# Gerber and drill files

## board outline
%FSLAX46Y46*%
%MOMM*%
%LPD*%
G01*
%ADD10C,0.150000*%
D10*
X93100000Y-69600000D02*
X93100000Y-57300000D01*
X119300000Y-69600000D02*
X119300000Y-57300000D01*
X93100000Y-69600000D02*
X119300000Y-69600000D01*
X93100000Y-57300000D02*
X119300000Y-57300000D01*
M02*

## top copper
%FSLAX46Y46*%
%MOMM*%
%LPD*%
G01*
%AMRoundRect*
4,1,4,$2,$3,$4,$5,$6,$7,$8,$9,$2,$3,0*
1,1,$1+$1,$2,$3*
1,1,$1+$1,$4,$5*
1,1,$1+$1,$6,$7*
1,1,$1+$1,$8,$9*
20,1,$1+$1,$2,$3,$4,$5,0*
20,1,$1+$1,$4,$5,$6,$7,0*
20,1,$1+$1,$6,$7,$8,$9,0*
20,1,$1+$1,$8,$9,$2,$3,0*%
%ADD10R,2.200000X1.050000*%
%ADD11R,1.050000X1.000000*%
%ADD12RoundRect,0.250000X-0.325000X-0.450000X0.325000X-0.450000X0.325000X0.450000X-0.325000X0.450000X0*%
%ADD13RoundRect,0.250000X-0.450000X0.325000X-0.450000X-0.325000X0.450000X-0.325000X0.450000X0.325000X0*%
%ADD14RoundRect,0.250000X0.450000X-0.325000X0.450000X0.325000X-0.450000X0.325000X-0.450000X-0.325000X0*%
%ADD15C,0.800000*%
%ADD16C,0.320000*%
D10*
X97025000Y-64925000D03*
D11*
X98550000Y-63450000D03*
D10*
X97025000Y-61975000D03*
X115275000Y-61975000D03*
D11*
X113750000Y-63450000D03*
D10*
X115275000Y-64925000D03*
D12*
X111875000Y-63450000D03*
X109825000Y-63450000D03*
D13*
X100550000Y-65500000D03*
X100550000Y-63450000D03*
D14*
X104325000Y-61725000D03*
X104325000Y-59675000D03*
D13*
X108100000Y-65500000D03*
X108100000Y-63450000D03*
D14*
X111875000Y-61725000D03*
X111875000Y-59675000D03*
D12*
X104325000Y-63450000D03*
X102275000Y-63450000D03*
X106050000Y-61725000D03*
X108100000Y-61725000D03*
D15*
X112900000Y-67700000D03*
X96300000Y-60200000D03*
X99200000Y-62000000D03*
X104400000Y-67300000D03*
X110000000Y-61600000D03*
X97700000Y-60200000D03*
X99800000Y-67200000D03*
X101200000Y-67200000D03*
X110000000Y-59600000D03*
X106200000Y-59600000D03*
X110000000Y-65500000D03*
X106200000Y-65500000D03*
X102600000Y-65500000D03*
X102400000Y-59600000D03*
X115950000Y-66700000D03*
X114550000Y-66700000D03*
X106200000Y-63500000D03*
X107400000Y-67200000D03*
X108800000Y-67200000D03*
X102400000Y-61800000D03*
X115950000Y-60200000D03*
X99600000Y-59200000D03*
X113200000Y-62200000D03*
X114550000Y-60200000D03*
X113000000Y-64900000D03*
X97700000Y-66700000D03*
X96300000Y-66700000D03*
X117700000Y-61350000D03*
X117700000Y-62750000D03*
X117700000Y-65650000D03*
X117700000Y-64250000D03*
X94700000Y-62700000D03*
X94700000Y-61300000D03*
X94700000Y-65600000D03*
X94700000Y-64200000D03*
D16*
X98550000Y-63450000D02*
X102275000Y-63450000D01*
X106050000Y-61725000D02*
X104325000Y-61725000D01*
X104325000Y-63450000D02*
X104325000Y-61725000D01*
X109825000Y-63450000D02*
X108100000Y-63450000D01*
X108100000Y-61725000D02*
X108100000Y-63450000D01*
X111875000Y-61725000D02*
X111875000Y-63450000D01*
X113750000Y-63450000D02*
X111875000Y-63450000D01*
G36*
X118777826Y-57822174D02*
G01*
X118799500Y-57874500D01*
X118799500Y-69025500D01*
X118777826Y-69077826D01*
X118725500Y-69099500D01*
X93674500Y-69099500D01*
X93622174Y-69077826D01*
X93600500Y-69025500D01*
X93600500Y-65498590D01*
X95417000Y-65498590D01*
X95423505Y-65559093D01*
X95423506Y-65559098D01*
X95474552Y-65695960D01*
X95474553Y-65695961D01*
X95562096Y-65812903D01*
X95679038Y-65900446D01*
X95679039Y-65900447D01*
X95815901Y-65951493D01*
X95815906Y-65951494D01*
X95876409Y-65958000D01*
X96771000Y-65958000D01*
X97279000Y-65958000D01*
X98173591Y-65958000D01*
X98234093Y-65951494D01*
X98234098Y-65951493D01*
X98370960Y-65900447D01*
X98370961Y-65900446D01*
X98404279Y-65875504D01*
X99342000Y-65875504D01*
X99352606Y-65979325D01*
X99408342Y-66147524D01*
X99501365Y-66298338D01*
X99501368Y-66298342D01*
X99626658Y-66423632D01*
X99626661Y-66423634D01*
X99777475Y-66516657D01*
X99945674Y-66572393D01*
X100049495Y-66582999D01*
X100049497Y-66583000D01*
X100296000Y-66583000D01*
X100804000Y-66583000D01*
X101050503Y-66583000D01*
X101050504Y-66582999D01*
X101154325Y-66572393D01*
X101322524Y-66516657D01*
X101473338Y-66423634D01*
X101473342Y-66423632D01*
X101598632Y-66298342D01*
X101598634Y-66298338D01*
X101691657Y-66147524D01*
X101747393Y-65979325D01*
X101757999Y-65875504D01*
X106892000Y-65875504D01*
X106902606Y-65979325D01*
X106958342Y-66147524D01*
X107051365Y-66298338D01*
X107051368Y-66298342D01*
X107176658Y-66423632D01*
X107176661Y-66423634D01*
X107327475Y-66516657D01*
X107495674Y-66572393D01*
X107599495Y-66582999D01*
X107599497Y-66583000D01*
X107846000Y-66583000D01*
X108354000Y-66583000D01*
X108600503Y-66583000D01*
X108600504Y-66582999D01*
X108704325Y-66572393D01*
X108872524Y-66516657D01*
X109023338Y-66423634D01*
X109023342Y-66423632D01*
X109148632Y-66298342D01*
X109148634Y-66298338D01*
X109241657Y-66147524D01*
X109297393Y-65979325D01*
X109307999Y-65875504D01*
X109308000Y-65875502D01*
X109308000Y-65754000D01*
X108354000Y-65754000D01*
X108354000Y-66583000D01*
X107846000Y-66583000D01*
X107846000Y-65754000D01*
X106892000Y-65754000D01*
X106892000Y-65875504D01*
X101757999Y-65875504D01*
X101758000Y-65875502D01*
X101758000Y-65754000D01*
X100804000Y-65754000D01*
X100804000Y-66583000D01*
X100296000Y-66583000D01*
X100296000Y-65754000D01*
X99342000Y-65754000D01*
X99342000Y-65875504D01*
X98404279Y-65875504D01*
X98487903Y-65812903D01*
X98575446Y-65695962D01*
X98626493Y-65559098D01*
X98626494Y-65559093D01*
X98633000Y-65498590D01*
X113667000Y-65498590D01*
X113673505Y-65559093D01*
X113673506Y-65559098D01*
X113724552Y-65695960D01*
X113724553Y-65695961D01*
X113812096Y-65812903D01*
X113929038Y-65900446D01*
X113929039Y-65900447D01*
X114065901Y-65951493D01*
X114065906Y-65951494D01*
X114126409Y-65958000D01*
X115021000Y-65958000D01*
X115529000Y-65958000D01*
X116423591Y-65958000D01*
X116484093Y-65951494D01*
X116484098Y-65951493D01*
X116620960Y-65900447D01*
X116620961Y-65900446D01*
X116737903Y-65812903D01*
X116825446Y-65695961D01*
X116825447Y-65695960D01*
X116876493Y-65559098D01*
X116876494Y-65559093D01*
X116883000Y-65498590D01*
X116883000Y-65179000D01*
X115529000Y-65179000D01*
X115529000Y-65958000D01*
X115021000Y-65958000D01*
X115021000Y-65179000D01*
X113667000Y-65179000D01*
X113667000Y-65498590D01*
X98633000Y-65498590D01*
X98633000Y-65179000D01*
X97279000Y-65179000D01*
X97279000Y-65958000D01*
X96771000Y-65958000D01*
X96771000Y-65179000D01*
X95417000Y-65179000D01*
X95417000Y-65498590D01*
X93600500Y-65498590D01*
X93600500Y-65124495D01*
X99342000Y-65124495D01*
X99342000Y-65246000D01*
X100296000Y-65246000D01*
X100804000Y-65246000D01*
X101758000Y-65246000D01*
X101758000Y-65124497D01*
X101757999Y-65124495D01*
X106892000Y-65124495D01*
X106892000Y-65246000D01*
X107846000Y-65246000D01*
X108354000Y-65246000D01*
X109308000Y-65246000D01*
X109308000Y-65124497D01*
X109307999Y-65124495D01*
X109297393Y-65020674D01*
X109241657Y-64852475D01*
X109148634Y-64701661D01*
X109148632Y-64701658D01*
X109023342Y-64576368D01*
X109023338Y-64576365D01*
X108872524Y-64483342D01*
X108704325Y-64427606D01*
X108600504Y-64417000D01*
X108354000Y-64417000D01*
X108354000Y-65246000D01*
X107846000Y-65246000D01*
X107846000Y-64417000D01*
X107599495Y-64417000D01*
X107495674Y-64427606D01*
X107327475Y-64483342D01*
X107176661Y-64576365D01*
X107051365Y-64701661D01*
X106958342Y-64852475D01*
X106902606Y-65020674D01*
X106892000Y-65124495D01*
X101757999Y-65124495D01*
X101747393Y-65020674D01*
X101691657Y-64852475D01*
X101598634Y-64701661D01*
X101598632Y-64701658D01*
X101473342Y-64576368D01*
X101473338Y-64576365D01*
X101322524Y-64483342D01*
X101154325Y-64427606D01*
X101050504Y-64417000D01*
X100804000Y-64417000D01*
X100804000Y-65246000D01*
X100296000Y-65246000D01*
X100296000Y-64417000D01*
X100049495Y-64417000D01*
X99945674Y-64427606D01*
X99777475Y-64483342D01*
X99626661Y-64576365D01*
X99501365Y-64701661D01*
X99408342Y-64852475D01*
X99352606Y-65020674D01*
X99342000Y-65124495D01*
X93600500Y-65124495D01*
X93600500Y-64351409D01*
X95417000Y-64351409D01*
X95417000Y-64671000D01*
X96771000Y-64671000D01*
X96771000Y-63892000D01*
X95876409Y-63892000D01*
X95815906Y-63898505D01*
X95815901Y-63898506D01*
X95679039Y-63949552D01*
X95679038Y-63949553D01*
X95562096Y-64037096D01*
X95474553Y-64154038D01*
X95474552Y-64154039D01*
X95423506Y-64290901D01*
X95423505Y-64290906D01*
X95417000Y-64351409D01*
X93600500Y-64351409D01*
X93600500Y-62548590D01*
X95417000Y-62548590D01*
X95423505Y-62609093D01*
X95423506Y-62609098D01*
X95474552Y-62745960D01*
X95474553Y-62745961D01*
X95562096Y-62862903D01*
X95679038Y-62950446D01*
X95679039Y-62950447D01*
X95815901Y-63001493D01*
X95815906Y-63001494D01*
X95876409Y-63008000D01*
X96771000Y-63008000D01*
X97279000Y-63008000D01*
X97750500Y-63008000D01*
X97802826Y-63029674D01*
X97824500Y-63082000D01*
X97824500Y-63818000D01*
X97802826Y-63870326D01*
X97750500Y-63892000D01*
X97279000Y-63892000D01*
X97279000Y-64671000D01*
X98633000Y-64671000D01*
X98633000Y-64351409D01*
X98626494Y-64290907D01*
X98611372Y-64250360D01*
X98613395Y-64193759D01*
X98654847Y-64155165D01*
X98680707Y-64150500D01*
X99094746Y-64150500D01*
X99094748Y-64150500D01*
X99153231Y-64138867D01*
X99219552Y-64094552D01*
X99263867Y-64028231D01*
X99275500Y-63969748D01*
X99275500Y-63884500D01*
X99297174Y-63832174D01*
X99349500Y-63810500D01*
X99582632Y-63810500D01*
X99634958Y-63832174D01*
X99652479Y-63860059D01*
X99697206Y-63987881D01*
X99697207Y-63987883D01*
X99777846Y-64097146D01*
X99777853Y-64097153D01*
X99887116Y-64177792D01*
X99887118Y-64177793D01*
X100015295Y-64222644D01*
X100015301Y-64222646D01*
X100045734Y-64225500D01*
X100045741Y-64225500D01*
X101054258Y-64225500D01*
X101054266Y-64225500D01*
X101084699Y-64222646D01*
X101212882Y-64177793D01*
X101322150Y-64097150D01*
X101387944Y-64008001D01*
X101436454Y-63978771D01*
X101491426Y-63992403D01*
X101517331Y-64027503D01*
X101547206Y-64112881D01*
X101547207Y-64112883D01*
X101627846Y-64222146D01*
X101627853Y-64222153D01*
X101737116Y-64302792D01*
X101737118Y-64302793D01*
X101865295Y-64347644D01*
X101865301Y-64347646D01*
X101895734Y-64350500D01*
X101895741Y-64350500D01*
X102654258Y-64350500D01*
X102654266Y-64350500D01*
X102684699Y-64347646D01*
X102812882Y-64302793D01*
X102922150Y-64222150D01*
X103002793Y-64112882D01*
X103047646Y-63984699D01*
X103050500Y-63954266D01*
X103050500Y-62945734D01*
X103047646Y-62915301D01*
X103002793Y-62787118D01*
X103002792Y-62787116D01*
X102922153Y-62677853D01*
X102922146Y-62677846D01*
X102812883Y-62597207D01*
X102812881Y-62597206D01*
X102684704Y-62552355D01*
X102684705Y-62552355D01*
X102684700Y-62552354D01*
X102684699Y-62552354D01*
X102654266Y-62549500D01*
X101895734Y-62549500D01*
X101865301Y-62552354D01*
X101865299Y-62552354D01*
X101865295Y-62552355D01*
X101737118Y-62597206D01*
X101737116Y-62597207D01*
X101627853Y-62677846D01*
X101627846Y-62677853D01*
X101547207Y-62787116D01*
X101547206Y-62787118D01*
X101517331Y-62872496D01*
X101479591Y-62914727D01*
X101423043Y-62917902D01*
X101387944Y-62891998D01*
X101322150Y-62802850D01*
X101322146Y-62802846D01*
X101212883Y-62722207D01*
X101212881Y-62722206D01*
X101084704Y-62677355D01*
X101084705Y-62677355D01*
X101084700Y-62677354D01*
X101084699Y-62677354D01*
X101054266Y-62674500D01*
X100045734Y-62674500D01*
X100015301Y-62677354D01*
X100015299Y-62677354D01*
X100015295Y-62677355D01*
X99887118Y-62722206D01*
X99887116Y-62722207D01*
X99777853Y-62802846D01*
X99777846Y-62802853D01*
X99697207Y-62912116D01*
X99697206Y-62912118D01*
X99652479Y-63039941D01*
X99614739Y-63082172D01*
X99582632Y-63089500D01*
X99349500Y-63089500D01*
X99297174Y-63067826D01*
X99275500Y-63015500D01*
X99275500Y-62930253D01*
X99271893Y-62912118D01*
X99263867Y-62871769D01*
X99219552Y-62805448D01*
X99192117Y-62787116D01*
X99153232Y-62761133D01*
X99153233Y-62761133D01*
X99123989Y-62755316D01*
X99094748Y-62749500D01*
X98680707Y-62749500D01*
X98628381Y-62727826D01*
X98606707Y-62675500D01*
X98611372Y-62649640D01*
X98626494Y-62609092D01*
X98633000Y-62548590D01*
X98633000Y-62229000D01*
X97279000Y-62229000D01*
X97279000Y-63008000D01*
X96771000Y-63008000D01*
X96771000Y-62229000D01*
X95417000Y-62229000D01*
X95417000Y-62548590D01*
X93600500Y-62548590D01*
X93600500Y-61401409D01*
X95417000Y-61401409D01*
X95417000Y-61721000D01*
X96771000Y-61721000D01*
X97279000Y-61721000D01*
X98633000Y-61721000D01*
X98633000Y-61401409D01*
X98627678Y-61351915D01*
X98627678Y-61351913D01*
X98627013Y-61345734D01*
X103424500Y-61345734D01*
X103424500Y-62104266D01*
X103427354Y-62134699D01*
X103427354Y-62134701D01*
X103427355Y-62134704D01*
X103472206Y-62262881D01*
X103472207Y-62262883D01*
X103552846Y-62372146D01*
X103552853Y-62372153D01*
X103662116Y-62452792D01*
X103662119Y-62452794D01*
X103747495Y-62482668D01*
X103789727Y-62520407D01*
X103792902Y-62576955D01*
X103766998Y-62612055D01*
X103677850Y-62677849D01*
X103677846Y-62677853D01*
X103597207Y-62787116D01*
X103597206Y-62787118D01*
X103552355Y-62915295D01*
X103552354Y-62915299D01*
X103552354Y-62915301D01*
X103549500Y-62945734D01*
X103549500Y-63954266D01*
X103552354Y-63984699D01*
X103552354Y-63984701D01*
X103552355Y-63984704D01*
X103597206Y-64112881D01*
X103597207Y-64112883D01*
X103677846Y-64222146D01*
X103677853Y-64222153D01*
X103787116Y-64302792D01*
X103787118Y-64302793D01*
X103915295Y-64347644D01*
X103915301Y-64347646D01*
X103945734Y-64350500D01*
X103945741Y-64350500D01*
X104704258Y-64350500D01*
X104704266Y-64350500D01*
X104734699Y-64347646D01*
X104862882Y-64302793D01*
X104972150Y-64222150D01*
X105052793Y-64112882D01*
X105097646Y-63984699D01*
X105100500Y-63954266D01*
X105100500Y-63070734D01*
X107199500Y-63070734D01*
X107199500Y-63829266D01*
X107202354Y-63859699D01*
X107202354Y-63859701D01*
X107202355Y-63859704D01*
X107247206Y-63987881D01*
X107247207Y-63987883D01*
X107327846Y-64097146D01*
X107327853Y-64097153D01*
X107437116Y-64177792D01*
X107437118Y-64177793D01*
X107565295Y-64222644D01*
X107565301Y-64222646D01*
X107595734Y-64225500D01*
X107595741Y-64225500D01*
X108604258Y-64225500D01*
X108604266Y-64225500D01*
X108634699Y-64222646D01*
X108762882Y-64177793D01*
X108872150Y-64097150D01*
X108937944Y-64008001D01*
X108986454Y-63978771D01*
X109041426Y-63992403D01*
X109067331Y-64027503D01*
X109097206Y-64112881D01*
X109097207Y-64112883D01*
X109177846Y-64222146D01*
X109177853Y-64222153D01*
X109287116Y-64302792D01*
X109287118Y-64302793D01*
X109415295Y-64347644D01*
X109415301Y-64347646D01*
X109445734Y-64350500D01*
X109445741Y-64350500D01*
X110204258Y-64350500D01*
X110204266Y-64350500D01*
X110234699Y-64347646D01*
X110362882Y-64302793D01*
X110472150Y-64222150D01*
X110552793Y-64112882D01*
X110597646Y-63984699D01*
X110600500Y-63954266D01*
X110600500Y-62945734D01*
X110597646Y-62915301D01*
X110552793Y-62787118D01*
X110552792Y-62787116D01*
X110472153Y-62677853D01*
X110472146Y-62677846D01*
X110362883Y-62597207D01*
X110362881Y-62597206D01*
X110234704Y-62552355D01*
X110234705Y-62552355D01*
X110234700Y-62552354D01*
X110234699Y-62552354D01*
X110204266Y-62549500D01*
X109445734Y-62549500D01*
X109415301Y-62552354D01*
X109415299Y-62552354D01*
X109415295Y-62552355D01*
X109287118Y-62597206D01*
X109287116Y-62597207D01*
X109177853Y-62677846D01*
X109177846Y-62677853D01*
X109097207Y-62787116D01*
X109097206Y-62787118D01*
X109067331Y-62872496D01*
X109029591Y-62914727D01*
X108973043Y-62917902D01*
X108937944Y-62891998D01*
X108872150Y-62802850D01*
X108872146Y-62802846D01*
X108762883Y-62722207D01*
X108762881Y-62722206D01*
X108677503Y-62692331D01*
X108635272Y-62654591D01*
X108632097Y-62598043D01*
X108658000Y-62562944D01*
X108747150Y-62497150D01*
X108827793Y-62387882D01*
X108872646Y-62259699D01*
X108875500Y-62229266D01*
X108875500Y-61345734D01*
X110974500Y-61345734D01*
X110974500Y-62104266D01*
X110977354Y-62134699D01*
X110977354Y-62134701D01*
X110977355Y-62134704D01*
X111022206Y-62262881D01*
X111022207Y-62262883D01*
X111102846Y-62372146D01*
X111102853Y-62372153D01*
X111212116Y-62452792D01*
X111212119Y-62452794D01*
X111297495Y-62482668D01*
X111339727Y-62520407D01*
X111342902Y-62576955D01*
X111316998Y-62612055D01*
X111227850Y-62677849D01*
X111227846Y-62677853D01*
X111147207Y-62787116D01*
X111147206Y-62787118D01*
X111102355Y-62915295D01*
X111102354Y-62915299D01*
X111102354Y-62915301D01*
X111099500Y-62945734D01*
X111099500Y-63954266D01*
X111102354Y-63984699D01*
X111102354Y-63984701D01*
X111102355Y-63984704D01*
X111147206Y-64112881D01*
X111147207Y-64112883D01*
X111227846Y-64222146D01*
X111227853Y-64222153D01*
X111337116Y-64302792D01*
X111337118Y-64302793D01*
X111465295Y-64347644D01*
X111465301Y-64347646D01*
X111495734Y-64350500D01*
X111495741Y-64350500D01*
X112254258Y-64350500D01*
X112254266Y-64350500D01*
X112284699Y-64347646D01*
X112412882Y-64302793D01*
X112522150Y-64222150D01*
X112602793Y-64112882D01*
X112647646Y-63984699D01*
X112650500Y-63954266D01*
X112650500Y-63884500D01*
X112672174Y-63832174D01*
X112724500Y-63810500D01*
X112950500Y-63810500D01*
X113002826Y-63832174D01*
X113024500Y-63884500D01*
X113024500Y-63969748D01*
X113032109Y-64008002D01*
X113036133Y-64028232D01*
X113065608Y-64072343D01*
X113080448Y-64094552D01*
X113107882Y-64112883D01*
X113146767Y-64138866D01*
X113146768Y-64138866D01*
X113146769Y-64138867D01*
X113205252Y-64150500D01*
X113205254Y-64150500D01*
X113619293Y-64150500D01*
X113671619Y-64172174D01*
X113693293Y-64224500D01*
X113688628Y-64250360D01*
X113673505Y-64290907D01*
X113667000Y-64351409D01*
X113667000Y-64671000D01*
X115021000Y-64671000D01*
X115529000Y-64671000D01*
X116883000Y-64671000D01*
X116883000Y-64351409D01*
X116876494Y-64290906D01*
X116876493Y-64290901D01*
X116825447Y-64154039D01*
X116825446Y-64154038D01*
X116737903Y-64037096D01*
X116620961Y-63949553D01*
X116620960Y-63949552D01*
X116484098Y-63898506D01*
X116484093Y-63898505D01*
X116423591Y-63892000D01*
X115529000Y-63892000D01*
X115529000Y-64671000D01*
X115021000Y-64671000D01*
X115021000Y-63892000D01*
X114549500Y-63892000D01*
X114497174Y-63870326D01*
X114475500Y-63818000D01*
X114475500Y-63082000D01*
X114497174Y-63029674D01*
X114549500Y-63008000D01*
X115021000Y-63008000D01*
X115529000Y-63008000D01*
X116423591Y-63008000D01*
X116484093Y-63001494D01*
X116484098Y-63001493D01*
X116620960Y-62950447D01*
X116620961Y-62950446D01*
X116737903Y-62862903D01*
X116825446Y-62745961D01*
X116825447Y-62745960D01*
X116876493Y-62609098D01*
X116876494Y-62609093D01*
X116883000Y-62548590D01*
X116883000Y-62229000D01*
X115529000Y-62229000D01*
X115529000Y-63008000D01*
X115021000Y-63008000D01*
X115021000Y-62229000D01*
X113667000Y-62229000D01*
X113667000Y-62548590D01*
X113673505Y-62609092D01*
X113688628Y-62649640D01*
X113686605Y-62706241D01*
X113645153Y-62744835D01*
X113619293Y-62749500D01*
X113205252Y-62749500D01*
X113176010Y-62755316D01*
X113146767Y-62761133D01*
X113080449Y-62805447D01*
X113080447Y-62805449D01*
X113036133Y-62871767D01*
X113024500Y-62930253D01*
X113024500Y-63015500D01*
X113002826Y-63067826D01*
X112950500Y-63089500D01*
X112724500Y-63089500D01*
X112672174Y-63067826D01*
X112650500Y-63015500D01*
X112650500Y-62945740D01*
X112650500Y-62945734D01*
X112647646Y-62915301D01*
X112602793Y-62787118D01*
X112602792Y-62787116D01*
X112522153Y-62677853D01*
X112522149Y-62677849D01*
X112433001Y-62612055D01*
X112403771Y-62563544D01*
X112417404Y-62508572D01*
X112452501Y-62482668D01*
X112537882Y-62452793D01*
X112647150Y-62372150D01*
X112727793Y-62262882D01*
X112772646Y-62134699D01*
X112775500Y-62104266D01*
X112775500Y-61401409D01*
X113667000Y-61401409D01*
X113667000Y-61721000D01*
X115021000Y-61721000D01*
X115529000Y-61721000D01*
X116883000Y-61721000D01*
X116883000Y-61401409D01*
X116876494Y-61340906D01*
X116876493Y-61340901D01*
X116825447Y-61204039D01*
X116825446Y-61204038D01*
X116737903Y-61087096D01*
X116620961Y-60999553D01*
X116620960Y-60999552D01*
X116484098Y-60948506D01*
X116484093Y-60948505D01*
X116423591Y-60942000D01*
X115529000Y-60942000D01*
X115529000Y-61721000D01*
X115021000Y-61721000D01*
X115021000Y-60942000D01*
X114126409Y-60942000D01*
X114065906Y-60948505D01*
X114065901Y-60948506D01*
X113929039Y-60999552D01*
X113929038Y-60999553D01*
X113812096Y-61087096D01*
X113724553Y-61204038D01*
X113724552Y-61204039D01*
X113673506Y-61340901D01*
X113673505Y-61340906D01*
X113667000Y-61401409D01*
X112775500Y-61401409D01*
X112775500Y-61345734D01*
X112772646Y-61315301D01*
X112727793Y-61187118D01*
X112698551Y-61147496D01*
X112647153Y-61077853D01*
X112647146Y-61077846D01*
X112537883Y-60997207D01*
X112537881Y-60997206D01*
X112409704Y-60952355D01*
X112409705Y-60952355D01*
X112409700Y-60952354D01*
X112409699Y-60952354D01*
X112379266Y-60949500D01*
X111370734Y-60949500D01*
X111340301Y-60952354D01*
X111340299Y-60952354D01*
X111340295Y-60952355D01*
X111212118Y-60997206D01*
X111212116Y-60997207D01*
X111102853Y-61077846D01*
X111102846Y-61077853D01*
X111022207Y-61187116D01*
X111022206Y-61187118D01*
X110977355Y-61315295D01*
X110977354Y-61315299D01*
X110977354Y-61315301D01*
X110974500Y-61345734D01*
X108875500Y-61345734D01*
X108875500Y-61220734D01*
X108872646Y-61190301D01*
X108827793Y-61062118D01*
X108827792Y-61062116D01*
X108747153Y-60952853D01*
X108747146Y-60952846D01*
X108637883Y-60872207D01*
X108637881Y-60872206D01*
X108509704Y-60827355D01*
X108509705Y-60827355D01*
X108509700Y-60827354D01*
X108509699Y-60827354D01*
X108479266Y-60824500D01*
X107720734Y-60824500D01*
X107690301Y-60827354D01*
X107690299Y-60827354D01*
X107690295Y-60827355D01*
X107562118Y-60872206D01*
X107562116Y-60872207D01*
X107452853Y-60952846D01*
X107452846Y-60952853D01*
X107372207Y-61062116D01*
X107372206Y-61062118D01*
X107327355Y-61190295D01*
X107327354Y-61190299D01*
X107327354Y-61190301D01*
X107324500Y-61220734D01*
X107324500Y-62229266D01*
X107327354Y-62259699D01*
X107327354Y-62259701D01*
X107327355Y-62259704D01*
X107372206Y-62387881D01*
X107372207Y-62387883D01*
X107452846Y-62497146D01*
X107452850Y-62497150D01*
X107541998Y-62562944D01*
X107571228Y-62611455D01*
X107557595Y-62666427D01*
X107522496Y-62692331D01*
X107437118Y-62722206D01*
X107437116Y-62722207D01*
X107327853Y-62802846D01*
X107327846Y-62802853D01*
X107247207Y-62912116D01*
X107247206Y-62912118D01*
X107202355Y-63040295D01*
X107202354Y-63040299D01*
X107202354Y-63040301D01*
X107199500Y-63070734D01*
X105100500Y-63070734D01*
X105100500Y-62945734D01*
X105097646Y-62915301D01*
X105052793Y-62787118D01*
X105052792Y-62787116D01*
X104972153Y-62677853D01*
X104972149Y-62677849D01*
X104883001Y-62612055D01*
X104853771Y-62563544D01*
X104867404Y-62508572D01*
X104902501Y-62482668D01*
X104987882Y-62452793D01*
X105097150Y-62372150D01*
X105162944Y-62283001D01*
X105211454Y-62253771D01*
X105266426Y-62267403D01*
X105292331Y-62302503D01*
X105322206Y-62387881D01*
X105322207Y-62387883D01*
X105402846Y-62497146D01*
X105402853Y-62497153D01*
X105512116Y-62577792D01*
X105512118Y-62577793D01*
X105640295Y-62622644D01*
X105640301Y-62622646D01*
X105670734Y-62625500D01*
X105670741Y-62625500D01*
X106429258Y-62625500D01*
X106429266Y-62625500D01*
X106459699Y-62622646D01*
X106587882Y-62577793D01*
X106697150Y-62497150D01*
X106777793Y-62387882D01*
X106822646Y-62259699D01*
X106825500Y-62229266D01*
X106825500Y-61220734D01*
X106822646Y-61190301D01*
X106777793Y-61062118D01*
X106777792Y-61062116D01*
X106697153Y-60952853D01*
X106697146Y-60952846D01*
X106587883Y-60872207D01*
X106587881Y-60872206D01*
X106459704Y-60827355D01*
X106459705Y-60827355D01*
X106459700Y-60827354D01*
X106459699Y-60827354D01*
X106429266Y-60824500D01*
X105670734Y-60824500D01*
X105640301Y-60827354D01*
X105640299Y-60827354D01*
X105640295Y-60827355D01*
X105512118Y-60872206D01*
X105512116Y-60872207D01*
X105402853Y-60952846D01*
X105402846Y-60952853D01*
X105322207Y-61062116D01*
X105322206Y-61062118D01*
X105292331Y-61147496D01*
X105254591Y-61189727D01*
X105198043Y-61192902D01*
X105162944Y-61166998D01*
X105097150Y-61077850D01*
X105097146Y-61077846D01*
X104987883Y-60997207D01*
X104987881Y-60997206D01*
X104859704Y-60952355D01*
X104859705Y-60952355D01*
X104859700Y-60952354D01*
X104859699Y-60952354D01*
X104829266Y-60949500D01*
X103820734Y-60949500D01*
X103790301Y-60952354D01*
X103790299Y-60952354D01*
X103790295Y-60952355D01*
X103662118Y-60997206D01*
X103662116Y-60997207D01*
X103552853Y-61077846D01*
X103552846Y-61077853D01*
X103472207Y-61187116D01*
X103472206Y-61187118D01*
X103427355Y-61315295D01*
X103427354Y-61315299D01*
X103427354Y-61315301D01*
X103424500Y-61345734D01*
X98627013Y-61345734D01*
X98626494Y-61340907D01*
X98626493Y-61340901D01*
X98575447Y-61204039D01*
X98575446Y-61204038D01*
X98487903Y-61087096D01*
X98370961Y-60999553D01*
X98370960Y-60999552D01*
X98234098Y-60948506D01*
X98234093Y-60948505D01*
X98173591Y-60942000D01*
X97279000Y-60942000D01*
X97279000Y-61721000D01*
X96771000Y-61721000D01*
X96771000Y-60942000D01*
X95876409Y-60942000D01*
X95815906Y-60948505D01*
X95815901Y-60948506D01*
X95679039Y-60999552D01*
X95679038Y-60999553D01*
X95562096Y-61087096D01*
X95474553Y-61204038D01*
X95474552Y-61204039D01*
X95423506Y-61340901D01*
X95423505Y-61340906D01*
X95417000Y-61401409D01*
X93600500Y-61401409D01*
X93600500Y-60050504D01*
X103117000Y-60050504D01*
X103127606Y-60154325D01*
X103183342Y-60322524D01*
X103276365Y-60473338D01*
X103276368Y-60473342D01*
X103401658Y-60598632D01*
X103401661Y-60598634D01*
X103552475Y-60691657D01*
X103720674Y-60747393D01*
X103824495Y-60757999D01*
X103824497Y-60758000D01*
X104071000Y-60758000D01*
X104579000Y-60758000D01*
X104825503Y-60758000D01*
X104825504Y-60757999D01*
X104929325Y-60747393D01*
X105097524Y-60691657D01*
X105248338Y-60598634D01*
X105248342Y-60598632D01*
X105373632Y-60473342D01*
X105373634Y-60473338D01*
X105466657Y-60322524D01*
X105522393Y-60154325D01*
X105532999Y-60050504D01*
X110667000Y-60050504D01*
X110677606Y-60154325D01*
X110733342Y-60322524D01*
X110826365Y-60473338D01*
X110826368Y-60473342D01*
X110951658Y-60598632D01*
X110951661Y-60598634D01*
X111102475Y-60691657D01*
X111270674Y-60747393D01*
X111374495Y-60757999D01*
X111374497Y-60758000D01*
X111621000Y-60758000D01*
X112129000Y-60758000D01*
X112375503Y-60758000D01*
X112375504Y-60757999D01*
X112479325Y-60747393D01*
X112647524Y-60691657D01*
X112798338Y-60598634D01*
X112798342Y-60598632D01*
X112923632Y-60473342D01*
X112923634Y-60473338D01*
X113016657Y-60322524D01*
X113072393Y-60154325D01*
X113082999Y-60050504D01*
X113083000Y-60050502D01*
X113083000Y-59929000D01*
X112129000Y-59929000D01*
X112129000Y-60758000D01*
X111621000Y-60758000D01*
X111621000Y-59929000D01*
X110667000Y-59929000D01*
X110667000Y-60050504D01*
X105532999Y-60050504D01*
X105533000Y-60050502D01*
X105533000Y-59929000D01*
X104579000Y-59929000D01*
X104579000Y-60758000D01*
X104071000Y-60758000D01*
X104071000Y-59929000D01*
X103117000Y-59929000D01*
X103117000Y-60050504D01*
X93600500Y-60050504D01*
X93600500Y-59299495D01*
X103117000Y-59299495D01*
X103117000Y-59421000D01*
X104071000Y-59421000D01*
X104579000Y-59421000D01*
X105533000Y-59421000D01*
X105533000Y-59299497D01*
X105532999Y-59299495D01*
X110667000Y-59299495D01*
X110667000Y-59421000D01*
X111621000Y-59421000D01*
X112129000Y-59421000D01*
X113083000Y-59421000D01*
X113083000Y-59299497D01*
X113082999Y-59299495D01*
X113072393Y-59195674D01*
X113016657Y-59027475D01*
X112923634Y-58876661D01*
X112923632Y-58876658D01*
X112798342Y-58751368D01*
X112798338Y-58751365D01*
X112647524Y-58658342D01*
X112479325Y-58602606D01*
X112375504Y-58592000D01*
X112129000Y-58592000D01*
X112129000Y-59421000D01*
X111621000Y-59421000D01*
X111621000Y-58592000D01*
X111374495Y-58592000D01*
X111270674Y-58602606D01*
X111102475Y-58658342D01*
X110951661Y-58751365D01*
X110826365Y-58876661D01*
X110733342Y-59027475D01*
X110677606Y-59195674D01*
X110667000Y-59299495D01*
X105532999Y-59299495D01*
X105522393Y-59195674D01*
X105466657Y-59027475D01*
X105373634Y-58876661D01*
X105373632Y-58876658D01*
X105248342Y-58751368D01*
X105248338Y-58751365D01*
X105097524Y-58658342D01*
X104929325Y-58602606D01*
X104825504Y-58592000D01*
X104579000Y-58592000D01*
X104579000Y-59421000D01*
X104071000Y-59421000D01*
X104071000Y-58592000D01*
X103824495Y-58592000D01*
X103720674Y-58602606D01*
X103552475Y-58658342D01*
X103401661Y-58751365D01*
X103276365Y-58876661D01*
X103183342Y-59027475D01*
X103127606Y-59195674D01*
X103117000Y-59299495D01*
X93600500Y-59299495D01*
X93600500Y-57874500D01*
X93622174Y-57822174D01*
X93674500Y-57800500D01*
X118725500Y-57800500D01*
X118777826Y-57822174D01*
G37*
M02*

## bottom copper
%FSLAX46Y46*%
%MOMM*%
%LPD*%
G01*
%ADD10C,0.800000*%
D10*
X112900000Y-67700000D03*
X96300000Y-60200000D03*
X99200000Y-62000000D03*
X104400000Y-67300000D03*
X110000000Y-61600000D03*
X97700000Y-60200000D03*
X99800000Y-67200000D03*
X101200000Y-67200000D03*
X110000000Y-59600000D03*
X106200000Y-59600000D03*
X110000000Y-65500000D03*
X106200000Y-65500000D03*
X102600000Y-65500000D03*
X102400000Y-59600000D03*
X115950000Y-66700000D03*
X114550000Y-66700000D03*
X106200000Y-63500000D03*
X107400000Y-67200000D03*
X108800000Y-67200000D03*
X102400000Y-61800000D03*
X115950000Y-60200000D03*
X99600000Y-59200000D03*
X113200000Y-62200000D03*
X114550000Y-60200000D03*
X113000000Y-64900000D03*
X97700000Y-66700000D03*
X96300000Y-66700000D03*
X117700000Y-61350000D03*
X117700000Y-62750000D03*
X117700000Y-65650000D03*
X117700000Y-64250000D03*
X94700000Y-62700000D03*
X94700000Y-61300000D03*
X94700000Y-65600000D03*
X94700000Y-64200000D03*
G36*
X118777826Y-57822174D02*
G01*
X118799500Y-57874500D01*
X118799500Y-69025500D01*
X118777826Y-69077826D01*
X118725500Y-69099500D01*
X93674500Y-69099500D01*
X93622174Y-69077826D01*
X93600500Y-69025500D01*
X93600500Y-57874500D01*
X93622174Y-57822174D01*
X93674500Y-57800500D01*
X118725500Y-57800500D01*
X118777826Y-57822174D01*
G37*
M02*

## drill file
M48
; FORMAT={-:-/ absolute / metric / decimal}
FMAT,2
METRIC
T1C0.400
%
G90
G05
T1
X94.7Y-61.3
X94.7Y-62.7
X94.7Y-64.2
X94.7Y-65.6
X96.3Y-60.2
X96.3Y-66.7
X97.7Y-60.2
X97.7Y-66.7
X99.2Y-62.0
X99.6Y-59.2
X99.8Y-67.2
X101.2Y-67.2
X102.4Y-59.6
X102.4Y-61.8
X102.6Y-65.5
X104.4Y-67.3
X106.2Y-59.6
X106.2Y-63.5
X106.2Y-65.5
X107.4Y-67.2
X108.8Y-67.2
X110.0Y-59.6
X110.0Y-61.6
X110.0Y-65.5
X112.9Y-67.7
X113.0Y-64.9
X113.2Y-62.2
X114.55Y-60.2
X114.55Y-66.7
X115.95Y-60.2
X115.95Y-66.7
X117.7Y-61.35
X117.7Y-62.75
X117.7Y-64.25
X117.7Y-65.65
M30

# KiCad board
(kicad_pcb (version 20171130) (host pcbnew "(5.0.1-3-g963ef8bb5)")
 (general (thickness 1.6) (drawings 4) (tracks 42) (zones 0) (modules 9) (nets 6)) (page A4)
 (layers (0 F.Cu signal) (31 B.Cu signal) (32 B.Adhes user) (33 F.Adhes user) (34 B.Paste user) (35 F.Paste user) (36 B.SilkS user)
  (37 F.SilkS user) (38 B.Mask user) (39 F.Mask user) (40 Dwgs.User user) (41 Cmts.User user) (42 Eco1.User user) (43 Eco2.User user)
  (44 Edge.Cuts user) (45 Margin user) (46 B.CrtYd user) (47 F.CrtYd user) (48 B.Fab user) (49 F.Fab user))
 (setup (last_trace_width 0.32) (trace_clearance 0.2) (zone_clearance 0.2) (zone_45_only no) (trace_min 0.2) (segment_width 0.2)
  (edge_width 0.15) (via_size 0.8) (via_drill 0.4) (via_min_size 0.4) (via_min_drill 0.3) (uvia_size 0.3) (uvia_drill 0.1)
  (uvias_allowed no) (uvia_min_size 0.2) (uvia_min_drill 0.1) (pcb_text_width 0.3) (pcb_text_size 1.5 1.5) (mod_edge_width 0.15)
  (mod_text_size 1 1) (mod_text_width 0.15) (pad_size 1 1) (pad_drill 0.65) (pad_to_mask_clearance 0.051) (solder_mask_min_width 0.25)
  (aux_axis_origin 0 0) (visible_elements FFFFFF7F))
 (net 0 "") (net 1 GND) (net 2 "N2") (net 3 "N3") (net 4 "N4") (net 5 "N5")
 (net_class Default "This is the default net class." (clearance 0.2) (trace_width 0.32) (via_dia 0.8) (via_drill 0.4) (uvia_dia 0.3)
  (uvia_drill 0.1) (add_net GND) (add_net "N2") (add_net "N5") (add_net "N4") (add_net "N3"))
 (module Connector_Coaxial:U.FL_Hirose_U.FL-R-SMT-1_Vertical (layer F.Cu) (at 97.5 63.45 180)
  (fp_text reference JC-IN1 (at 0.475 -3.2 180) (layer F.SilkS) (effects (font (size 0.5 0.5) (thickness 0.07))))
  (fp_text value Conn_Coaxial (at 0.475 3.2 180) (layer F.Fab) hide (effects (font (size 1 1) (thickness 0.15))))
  (pad 2 smd rect (at 0.475 -1.475 180) (size 2.2 1.05) (layers F.Cu F.Paste F.Mask) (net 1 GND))
  (pad 1 smd rect (at -1.05 0 180) (size 1.05 1) (layers F.Cu F.Paste F.Mask) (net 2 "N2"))
  (pad 2 smd rect (at 0.475 1.475 180) (size 2.2 1.05) (layers F.Cu F.Paste F.Mask) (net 1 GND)))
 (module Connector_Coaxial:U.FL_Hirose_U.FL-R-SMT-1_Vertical (layer F.Cu) (at 114.8 63.45)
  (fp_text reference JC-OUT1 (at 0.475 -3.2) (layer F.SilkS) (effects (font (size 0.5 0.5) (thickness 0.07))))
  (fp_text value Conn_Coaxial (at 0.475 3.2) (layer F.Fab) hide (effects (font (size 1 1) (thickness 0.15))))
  (pad 2 smd rect (at 0.475 -1.475) (size 2.2 1.05) (layers F.Cu F.Paste F.Mask) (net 1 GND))
  (pad 1 smd rect (at -1.05 0) (size 1.05 1) (layers F.Cu F.Paste F.Mask) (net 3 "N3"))
  (pad 2 smd rect (at 0.475 1.475) (size 2.2 1.05) (layers F.Cu F.Paste F.Mask) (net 1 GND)))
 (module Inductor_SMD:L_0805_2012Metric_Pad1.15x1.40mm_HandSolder (layer F.Cu) (at 110.85 63.45)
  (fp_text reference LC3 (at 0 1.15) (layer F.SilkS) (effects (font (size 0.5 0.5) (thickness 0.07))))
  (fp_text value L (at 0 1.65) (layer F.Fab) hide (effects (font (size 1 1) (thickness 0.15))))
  (pad 2 smd roundrect (at 1.025 0) (size 1.15 1.4) (layers F.Cu F.Paste F.Mask) (roundrect_rratio 0.217391) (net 3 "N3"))
  (pad 1 smd roundrect (at -1.025 0) (size 1.15 1.4) (layers F.Cu F.Paste F.Mask) (roundrect_rratio 0.217391) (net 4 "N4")))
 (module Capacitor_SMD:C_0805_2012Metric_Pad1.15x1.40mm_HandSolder (layer F.Cu) (at 100.55 64.475 270)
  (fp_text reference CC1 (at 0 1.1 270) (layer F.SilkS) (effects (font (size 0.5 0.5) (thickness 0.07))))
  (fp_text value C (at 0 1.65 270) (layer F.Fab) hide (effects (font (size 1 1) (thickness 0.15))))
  (pad 2 smd roundrect (at 1.025 0 270) (size 1.15 1.4) (layers F.Cu F.Paste F.Mask) (roundrect_rratio 0.217391) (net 1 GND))
  (pad 1 smd roundrect (at -1.025 0 270) (size 1.15 1.4) (layers F.Cu F.Paste F.Mask) (roundrect_rratio 0.217391) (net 2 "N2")))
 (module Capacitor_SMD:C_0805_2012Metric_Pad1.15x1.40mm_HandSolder (layer F.Cu) (at 104.325 60.7 90)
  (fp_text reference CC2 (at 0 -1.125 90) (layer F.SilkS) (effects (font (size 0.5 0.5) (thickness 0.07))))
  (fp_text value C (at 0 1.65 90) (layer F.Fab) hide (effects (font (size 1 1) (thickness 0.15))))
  (pad 1 smd roundrect (at -1.025 0 90) (size 1.15 1.4) (layers F.Cu F.Paste F.Mask) (roundrect_rratio 0.217391) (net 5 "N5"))
  (pad 2 smd roundrect (at 1.025 0 90) (size 1.15 1.4) (layers F.Cu F.Paste F.Mask) (roundrect_rratio 0.217391) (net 1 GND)))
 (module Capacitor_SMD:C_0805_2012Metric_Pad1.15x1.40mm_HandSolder (layer F.Cu) (at 108.1 64.475 270)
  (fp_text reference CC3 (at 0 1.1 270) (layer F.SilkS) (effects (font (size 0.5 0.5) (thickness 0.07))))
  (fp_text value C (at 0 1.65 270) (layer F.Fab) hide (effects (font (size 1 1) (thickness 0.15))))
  (pad 2 smd roundrect (at 1.025 0 270) (size 1.15 1.4) (layers F.Cu F.Paste F.Mask) (roundrect_rratio 0.217391) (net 1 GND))
  (pad 1 smd roundrect (at -1.025 0 270) (size 1.15 1.4) (layers F.Cu F.Paste F.Mask) (roundrect_rratio 0.217391) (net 4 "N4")))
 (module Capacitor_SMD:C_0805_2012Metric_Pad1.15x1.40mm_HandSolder (layer F.Cu) (at 111.875 60.7 90)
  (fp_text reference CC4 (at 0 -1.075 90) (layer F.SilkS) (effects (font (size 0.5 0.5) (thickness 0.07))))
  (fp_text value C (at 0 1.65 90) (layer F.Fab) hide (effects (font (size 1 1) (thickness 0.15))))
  (pad 1 smd roundrect (at -1.025 0 90) (size 1.15 1.4) (layers F.Cu F.Paste F.Mask) (roundrect_rratio 0.217391) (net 3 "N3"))
  (pad 2 smd roundrect (at 1.025 0 90) (size 1.15 1.4) (layers F.Cu F.Paste F.Mask) (roundrect_rratio 0.217391) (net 1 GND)))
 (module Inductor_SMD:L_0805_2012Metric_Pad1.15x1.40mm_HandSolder (layer F.Cu) (at 103.3 63.45)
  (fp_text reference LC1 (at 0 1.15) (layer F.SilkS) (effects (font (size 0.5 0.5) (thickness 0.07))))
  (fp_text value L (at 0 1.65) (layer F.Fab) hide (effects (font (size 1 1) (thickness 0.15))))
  (pad 2 smd roundrect (at 1.025 0) (size 1.15 1.4) (layers F.Cu F.Paste F.Mask) (roundrect_rratio 0.217391) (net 5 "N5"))
  (pad 1 smd roundrect (at -1.025 0) (size 1.15 1.4) (layers F.Cu F.Paste F.Mask) (roundrect_rratio 0.217391) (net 2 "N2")))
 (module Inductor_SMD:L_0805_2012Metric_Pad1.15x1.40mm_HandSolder (layer F.Cu) (at 107.075 61.725)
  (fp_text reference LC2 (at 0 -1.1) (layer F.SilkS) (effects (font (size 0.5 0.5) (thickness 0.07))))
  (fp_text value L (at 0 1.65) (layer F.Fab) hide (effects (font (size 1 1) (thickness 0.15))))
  (pad 1 smd roundrect (at -1.025 0) (size 1.15 1.4) (layers F.Cu F.Paste F.Mask) (roundrect_rratio 0.217391) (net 5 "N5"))
  (pad 2 smd roundrect (at 1.025 0) (size 1.15 1.4) (layers F.Cu F.Paste F.Mask) (roundrect_rratio 0.217391) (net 4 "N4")))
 (gr_line (start 93.1 69.6) (end 93.1 57.3) (layer Edge.Cuts) (width 0.15))
 (gr_line (start 119.3 69.6) (end 119.3 57.3) (layer Edge.Cuts) (width 0.15))
 (gr_line (start 93.1 69.6) (end 119.3 69.6) (layer Edge.Cuts) (width 0.15))
 (gr_line (start 93.1 57.3) (end 119.3 57.3) (layer Edge.Cuts) (width 0.15))
 (via (at 112.9 67.7) (size 0.8) (drill 0.4) (layers F.Cu B.Cu) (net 1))
 (via (at 96.3 60.2) (size 0.8) (drill 0.4) (layers F.Cu B.Cu) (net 1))
 (via (at 99.2 62) (size 0.8) (drill 0.4) (layers F.Cu B.Cu) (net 1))
 (via (at 104.4 67.3) (size 0.8) (drill 0.4) (layers F.Cu B.Cu) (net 1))
 (via (at 110 61.6) (size 0.8) (drill 0.4) (layers F.Cu B.Cu) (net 1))
 (via (at 97.7 60.2) (size 0.8) (drill 0.4) (layers F.Cu B.Cu) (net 1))
 (via (at 99.8 67.2) (size 0.8) (drill 0.4) (layers F.Cu B.Cu) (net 1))
 (via (at 101.2 67.2) (size 0.8) (drill 0.4) (layers F.Cu B.Cu) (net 1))
 (via (at 110 59.6) (size 0.8) (drill 0.4) (layers F.Cu B.Cu) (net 1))
 (via (at 106.2 59.6) (size 0.8) (drill 0.4) (layers F.Cu B.Cu) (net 1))
 (via (at 110 65.5) (size 0.8) (drill 0.4) (layers F.Cu B.Cu) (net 1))
 (via (at 106.2 65.5) (size 0.8) (drill 0.4) (layers F.Cu B.Cu) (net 1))
 (via (at 102.6 65.5) (size 0.8) (drill 0.4) (layers F.Cu B.Cu) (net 1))
 (via (at 102.4 59.6) (size 0.8) (drill 0.4) (layers F.Cu B.Cu) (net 1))
 (via (at 115.95 66.7) (size 0.8) (drill 0.4) (layers F.Cu B.Cu) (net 1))
 (via (at 114.55 66.7) (size 0.8) (drill 0.4) (layers F.Cu B.Cu) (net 1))
 (via (at 106.2 63.5) (size 0.8) (drill 0.4) (layers F.Cu B.Cu) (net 1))
 (via (at 107.4 67.2) (size 0.8) (drill 0.4) (layers F.Cu B.Cu) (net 1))
 (via (at 108.8 67.2) (size 0.8) (drill 0.4) (layers F.Cu B.Cu) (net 1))
 (via (at 102.4 61.8) (size 0.8) (drill 0.4) (layers F.Cu B.Cu) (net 1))
 (via (at 115.95 60.2) (size 0.8) (drill 0.4) (layers F.Cu B.Cu) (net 1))
 (via (at 99.6 59.2) (size 0.8) (drill 0.4) (layers F.Cu B.Cu) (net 1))
 (via (at 113.2 62.2) (size 0.8) (drill 0.4) (layers F.Cu B.Cu) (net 1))
 (via (at 114.55 60.2) (size 0.8) (drill 0.4) (layers F.Cu B.Cu) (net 1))
 (via (at 113 64.9) (size 0.8) (drill 0.4) (layers F.Cu B.Cu) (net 1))
 (via (at 97.7 66.7) (size 0.8) (drill 0.4) (layers F.Cu B.Cu) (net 1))
 (via (at 96.3 66.7) (size 0.8) (drill 0.4) (layers F.Cu B.Cu) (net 1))
 (via (at 117.7 61.35) (size 0.8) (drill 0.4) (layers F.Cu B.Cu) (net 1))
 (via (at 117.7 62.75) (size 0.8) (drill 0.4) (layers F.Cu B.Cu) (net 1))
 (via (at 117.7 65.65) (size 0.8) (drill 0.4) (layers F.Cu B.Cu) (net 1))
 (via (at 117.7 64.25) (size 0.8) (drill 0.4) (layers F.Cu B.Cu) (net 1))
 (via (at 94.7 62.7) (size 0.8) (drill 0.4) (layers F.Cu B.Cu) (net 1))
 (via (at 94.7 61.3) (size 0.8) (drill 0.4) (layers F.Cu B.Cu) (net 1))
 (via (at 94.7 65.6) (size 0.8) (drill 0.4) (layers F.Cu B.Cu) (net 1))
 (via (at 94.7 64.2) (size 0.8) (drill 0.4) (layers F.Cu B.Cu) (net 1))
 (segment (start 98.55 63.45) (end 102.275 63.45) (width 0.32) (layer F.Cu) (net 2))
 (segment (start 106.05 61.725) (end 104.325 61.725) (width 0.32) (layer F.Cu) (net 5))
 (segment (start 104.325 63.45) (end 104.325 61.725) (width 0.32) (layer F.Cu) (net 5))
 (segment (start 109.825 63.45) (end 108.1 63.45) (width 0.32) (layer F.Cu) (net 4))
 (segment (start 108.1 61.725) (end 108.1 63.45) (width 0.32) (layer F.Cu) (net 4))
 (segment (start 111.875 61.725) (end 111.875 63.45) (width 0.32) (layer F.Cu) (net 3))
 (segment (start 113.75 63.45) (end 111.875 63.45) (width 0.32) (layer F.Cu) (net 3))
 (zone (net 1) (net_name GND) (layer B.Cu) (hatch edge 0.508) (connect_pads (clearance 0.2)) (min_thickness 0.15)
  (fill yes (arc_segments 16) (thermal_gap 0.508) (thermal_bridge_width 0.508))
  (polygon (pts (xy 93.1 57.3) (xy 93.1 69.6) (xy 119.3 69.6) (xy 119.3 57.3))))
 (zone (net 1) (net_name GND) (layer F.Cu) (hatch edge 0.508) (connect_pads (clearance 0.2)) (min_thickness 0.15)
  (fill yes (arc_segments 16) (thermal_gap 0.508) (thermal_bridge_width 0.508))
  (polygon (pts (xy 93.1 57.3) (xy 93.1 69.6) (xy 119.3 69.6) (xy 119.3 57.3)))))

